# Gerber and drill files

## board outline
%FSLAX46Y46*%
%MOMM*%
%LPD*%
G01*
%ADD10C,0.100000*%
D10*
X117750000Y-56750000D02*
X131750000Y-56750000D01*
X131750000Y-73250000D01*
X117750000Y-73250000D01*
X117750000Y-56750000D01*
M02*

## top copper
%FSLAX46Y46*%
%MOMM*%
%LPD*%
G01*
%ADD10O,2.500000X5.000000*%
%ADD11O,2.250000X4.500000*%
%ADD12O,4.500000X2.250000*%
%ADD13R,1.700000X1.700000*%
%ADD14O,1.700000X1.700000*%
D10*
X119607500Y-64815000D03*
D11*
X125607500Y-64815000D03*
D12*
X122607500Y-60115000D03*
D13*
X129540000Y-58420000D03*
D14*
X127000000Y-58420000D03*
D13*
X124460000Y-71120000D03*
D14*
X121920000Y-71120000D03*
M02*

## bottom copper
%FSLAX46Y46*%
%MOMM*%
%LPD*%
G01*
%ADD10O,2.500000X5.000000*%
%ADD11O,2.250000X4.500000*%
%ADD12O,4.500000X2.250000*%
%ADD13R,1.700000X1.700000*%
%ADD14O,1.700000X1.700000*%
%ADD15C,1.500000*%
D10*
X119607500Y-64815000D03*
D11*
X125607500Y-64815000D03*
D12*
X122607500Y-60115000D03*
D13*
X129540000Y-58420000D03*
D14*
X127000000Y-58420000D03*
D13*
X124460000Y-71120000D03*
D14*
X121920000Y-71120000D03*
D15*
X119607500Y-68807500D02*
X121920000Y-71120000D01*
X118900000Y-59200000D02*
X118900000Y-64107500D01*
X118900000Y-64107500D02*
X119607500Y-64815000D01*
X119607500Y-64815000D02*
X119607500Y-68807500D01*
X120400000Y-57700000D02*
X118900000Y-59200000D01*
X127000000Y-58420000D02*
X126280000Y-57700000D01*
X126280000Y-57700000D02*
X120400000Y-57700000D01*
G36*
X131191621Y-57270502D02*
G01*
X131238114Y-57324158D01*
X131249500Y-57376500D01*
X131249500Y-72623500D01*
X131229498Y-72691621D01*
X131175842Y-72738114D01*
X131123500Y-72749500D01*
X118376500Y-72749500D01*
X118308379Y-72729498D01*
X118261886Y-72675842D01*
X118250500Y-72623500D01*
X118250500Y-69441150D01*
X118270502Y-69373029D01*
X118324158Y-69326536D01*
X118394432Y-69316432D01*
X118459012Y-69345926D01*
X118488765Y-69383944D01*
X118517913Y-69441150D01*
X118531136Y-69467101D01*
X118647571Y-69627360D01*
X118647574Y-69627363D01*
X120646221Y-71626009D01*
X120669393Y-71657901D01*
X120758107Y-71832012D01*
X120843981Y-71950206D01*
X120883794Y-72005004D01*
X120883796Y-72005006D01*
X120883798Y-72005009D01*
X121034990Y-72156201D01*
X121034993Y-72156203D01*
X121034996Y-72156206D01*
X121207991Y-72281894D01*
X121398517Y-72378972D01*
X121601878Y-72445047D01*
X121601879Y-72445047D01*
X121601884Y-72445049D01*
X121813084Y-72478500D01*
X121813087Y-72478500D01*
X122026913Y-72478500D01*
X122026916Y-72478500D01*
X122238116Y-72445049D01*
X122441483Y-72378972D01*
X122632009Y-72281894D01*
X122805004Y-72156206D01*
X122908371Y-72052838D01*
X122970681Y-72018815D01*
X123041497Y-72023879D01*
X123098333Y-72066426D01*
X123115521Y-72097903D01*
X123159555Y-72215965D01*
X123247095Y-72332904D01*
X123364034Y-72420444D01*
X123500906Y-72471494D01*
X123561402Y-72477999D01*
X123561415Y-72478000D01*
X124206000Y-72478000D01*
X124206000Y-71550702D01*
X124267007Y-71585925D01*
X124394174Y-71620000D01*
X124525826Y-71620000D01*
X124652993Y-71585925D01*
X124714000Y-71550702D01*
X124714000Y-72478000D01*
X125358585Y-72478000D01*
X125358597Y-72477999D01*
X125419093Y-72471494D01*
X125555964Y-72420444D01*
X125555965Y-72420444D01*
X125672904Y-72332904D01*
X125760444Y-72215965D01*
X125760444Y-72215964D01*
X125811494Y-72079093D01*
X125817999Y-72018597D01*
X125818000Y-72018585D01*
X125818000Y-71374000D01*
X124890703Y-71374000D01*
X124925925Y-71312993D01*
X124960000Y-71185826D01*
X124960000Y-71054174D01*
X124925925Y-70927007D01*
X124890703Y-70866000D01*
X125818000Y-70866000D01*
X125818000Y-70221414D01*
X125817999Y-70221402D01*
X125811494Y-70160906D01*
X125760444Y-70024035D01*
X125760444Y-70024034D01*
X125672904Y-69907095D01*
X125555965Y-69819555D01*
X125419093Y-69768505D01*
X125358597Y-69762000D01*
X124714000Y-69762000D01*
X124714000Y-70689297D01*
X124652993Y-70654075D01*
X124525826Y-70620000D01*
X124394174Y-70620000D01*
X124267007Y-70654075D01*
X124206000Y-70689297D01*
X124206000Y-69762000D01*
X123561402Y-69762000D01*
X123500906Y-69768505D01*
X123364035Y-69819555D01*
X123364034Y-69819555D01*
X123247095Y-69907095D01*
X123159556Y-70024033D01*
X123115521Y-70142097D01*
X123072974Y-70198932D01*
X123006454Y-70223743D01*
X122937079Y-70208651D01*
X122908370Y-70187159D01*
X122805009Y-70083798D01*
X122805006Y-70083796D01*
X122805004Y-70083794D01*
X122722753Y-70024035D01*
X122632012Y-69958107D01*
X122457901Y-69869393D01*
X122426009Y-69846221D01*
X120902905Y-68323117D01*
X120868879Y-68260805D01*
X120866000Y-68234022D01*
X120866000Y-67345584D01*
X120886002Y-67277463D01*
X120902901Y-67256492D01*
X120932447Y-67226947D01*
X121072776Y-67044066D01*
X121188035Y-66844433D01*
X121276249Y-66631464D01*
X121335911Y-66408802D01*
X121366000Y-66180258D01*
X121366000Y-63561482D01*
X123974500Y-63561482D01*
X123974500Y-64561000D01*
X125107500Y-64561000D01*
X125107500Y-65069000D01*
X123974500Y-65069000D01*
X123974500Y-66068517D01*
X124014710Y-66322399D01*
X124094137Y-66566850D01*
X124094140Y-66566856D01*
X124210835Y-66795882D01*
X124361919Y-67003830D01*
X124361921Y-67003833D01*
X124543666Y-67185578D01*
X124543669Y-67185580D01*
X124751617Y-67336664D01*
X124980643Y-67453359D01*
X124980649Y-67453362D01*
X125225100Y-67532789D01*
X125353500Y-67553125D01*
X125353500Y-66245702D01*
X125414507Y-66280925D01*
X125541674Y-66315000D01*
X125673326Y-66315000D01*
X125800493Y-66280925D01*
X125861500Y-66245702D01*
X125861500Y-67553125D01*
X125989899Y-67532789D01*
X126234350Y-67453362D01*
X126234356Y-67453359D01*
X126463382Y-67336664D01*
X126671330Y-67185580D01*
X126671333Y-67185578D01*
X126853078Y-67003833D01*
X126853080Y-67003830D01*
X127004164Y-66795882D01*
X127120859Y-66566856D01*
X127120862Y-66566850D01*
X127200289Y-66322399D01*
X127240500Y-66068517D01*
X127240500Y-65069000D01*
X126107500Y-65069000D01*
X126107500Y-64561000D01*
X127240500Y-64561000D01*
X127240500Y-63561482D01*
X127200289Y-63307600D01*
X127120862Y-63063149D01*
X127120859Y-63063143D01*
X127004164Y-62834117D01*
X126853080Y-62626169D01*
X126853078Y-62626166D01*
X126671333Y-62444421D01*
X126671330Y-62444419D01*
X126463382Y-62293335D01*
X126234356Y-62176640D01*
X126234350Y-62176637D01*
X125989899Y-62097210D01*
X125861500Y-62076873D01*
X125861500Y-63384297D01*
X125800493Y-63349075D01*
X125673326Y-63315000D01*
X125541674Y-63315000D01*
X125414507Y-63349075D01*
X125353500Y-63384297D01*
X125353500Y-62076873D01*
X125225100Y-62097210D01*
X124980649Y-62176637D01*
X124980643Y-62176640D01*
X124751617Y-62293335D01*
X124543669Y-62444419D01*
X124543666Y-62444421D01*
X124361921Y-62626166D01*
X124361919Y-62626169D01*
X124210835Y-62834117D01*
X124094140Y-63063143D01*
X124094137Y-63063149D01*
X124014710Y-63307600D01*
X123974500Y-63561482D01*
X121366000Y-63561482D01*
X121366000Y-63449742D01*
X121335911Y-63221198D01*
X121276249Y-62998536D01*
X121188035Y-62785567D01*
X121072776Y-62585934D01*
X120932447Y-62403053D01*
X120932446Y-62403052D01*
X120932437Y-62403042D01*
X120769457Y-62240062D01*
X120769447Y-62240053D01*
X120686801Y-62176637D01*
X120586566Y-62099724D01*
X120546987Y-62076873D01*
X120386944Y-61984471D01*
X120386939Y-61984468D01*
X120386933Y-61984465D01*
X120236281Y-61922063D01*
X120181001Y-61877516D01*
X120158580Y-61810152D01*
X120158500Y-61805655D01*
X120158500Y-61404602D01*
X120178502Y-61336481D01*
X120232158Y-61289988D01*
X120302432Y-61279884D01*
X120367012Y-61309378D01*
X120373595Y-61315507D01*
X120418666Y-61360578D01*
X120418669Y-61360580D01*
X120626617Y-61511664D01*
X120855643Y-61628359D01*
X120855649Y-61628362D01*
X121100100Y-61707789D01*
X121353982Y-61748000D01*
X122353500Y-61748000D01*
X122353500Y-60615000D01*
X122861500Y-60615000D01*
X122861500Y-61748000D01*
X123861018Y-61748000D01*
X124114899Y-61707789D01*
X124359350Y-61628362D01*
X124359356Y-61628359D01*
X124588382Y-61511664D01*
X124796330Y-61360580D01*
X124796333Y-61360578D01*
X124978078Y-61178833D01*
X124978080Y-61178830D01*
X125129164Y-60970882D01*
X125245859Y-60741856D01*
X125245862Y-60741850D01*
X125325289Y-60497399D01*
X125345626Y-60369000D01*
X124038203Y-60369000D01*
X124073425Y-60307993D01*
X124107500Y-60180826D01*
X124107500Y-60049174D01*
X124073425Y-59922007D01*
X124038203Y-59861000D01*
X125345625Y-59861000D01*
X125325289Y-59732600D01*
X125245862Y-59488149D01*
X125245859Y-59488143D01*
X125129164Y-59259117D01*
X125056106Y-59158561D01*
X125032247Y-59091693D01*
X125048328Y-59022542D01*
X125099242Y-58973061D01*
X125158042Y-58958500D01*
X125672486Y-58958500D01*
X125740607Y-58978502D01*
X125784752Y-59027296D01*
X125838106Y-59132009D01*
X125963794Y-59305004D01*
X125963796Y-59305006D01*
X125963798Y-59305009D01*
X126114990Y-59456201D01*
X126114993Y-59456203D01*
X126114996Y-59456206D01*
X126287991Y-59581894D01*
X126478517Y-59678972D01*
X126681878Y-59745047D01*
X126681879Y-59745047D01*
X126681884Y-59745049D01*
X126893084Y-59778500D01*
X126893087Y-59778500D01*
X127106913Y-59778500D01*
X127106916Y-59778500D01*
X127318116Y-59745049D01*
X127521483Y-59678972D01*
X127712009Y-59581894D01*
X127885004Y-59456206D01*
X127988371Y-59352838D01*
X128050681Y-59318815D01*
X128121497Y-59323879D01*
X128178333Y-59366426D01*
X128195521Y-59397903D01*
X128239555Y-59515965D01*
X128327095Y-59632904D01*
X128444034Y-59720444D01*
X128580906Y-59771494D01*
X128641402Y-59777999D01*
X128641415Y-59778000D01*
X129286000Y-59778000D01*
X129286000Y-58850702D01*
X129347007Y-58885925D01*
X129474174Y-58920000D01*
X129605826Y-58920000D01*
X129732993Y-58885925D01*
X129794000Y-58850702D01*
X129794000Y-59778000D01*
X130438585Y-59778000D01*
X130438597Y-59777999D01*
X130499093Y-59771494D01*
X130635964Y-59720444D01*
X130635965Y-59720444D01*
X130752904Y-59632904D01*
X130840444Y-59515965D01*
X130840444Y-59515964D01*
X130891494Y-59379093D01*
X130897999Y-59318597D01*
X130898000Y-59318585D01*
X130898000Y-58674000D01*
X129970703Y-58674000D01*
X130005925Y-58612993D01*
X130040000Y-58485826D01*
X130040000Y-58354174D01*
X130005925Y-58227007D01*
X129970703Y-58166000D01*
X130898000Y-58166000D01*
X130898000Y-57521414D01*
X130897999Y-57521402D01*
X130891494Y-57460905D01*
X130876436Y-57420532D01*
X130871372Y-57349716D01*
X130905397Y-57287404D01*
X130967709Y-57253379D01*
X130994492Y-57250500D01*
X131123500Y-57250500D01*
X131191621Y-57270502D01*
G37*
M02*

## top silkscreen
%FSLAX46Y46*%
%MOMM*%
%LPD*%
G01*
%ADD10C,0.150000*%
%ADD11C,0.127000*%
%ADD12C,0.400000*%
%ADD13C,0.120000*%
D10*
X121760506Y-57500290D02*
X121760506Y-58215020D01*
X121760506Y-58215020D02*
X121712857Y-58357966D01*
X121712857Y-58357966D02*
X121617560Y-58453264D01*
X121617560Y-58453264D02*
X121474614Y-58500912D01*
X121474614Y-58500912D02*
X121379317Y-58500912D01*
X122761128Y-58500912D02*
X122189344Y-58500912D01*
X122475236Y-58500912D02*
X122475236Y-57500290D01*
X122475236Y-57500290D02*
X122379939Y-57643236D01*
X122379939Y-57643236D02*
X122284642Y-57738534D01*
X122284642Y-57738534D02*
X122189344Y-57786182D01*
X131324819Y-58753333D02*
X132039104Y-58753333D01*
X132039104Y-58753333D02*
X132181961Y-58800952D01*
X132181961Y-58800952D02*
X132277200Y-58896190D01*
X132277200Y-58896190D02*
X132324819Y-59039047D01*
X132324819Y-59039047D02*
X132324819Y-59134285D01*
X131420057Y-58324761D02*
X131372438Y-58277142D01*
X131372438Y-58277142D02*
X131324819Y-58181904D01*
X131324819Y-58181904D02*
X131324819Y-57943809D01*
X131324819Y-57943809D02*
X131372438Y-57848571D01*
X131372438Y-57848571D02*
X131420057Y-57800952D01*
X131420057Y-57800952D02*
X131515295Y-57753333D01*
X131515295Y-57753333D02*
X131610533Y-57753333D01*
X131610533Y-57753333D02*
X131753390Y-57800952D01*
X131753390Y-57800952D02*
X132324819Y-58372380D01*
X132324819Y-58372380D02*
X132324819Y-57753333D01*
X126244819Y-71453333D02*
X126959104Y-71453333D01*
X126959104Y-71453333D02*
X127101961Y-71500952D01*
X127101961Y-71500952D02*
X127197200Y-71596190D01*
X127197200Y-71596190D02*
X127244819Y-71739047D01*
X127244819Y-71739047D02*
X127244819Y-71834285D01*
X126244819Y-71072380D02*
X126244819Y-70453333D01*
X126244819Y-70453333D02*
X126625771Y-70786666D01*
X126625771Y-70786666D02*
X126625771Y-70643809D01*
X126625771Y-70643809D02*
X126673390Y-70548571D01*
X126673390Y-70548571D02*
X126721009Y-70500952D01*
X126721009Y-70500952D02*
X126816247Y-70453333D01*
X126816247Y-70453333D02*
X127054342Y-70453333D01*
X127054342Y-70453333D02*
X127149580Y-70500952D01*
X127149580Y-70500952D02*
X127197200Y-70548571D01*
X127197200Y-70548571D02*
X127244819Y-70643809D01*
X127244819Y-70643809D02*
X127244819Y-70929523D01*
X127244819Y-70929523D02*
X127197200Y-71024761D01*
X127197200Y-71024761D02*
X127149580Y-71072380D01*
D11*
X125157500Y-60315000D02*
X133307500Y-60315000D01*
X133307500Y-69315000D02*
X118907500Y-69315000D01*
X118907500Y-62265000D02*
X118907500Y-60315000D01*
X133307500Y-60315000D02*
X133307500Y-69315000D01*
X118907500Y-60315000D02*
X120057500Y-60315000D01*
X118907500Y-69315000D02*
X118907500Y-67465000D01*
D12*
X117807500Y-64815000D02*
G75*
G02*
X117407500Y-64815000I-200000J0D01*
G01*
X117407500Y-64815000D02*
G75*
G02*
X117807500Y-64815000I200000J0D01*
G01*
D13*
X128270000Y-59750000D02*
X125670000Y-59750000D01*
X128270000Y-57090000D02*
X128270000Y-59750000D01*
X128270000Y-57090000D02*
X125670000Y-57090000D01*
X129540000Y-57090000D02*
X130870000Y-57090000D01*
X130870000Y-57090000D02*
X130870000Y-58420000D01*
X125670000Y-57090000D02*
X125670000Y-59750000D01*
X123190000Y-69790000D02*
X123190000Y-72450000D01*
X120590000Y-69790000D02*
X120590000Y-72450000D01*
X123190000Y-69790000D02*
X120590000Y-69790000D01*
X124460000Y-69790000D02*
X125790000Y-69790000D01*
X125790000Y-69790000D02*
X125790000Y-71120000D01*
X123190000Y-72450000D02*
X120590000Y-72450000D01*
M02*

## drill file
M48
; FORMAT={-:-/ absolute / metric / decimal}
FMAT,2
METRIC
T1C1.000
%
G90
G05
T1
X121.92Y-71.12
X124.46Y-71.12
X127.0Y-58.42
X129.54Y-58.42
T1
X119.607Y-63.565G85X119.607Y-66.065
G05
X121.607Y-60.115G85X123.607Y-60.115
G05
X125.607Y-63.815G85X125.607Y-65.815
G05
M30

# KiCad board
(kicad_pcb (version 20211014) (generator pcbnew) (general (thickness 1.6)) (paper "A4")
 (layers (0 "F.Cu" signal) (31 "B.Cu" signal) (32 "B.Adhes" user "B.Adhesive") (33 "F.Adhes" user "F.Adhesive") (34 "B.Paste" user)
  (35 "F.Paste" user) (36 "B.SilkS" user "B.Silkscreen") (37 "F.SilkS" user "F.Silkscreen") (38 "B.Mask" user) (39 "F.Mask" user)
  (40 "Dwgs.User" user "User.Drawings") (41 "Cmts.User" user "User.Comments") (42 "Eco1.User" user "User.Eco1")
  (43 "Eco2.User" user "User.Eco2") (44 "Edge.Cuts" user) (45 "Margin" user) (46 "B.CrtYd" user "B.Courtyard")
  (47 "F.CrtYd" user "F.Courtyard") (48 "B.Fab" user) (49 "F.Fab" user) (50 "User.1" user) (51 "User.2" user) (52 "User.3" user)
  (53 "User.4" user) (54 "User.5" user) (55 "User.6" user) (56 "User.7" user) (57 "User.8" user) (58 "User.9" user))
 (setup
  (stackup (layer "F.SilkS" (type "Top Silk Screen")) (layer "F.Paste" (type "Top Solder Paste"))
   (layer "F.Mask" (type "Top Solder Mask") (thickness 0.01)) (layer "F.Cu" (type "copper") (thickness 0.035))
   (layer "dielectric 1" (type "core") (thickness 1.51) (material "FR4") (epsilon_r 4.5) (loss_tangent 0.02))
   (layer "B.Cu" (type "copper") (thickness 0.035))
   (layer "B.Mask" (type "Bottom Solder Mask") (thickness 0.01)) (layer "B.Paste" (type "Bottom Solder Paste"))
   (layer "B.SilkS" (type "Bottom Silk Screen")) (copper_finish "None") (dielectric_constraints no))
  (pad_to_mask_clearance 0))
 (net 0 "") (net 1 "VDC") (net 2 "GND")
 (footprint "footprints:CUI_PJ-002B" (layer "F.Cu") (at 119.6075 64.815)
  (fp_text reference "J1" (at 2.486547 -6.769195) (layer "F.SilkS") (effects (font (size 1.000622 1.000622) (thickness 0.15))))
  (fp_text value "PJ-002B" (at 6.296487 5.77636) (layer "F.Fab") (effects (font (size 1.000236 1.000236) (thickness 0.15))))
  (fp_line (start 5.55 -4.5) (end 13.7 -4.5) (layer "F.SilkS") (width 0.127))
  (fp_line (start 13.7 4.5) (end -0.7 4.5) (layer "F.SilkS") (width 0.127))
  (fp_line (start -0.7 -2.55) (end -0.7 -4.5) (layer "F.SilkS") (width 0.127))
  (fp_line (start 13.7 -4.5) (end 13.7 4.5) (layer "F.SilkS") (width 0.127))
  (fp_line (start -0.7 -4.5) (end 0.45 -4.5) (layer "F.SilkS") (width 0.127))
  (fp_line (start -0.7 4.5) (end -0.7 2.65) (layer "F.SilkS") (width 0.127))
  (fp_circle (center -2 0) (end -1.8 0) (layer "F.SilkS") (width 0.4) (fill none))
  (pad "1" thru_hole oval locked (at 0 0) (size 2.5 5) (drill oval 1 3.5) (layers *.Cu *.Mask) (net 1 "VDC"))
  (pad "2" thru_hole oval locked (at 6 0) (size 2.25 4.5) (drill oval 1 3) (layers *.Cu *.Mask) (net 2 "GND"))
  (pad "3" thru_hole oval locked (at 3 -4.7) (size 4.5 2.25) (drill oval 3 1) (layers *.Cu *.Mask) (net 2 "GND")))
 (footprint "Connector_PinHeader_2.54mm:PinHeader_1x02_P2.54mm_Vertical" (layer "F.Cu") (at 129.54 58.42 -90)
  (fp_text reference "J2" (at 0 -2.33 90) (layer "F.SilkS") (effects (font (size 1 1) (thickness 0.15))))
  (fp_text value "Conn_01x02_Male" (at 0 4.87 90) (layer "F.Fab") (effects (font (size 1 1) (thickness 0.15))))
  (fp_line (start 1.33 1.27) (end 1.33 3.87) (layer "F.SilkS") (width 0.12))
  (fp_line (start -1.33 1.27) (end 1.33 1.27) (layer "F.SilkS") (width 0.12))
  (fp_line (start -1.33 1.27) (end -1.33 3.87) (layer "F.SilkS") (width 0.12))
  (fp_line (start -1.33 0) (end -1.33 -1.33) (layer "F.SilkS") (width 0.12))
  (fp_line (start -1.33 -1.33) (end 0 -1.33) (layer "F.SilkS") (width 0.12))
  (fp_line (start -1.33 3.87) (end 1.33 3.87) (layer "F.SilkS") (width 0.12))
  (pad "1" thru_hole rect (at 0 0 270) (size 1.7 1.7) (drill 1) (layers *.Cu *.Mask) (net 2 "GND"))
  (pad "2" thru_hole oval (at 0 2.54 270) (size 1.7 1.7) (drill 1) (layers *.Cu *.Mask) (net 1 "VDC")))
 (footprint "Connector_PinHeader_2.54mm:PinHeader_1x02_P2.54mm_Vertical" (layer "F.Cu") (at 124.46 71.12 -90)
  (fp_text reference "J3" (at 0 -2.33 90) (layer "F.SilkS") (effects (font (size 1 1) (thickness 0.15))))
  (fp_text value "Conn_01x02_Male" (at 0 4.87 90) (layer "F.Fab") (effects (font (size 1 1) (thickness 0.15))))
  (fp_line (start -1.33 1.27) (end 1.33 1.27) (layer "F.SilkS") (width 0.12))
  (fp_line (start -1.33 3.87) (end 1.33 3.87) (layer "F.SilkS") (width 0.12))
  (fp_line (start -1.33 1.27) (end -1.33 3.87) (layer "F.SilkS") (width 0.12))
  (fp_line (start -1.33 0) (end -1.33 -1.33) (layer "F.SilkS") (width 0.12))
  (fp_line (start -1.33 -1.33) (end 0 -1.33) (layer "F.SilkS") (width 0.12))
  (fp_line (start 1.33 1.27) (end 1.33 3.87) (layer "F.SilkS") (width 0.12))
  (pad "1" thru_hole rect (at 0 0 270) (size 1.7 1.7) (drill 1) (layers *.Cu *.Mask) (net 2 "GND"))
  (pad "2" thru_hole oval (at 0 2.54 270) (size 1.7 1.7) (drill 1) (layers *.Cu *.Mask) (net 1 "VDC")))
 (gr_rect (start 117.75 56.75) (end 131.75 73.25) (layer "Edge.Cuts") (width 0.1) (fill none))
 (segment (start 119.6075 68.8075) (end 121.92 71.12) (width 1.5) (layer "B.Cu") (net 1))
 (segment (start 118.9 59.2) (end 118.9 64.1075) (width 1.5) (layer "B.Cu") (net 1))
 (segment (start 118.9 64.1075) (end 119.6075 64.815) (width 1.5) (layer "B.Cu") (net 1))
 (segment (start 119.6075 64.815) (end 119.6075 68.8075) (width 1.5) (layer "B.Cu") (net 1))
 (segment (start 120.4 57.7) (end 118.9 59.2) (width 1.5) (layer "B.Cu") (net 1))
 (segment (start 127 58.42) (end 126.28 57.7) (width 1.5) (layer "B.Cu") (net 1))
 (segment (start 126.28 57.7) (end 120.4 57.7) (width 1.5) (layer "B.Cu") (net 1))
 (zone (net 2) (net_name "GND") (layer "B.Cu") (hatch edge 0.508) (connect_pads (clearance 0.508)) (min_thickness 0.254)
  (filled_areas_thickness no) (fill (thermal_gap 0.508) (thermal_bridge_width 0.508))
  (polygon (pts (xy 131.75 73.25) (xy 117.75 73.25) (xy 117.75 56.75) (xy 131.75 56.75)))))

